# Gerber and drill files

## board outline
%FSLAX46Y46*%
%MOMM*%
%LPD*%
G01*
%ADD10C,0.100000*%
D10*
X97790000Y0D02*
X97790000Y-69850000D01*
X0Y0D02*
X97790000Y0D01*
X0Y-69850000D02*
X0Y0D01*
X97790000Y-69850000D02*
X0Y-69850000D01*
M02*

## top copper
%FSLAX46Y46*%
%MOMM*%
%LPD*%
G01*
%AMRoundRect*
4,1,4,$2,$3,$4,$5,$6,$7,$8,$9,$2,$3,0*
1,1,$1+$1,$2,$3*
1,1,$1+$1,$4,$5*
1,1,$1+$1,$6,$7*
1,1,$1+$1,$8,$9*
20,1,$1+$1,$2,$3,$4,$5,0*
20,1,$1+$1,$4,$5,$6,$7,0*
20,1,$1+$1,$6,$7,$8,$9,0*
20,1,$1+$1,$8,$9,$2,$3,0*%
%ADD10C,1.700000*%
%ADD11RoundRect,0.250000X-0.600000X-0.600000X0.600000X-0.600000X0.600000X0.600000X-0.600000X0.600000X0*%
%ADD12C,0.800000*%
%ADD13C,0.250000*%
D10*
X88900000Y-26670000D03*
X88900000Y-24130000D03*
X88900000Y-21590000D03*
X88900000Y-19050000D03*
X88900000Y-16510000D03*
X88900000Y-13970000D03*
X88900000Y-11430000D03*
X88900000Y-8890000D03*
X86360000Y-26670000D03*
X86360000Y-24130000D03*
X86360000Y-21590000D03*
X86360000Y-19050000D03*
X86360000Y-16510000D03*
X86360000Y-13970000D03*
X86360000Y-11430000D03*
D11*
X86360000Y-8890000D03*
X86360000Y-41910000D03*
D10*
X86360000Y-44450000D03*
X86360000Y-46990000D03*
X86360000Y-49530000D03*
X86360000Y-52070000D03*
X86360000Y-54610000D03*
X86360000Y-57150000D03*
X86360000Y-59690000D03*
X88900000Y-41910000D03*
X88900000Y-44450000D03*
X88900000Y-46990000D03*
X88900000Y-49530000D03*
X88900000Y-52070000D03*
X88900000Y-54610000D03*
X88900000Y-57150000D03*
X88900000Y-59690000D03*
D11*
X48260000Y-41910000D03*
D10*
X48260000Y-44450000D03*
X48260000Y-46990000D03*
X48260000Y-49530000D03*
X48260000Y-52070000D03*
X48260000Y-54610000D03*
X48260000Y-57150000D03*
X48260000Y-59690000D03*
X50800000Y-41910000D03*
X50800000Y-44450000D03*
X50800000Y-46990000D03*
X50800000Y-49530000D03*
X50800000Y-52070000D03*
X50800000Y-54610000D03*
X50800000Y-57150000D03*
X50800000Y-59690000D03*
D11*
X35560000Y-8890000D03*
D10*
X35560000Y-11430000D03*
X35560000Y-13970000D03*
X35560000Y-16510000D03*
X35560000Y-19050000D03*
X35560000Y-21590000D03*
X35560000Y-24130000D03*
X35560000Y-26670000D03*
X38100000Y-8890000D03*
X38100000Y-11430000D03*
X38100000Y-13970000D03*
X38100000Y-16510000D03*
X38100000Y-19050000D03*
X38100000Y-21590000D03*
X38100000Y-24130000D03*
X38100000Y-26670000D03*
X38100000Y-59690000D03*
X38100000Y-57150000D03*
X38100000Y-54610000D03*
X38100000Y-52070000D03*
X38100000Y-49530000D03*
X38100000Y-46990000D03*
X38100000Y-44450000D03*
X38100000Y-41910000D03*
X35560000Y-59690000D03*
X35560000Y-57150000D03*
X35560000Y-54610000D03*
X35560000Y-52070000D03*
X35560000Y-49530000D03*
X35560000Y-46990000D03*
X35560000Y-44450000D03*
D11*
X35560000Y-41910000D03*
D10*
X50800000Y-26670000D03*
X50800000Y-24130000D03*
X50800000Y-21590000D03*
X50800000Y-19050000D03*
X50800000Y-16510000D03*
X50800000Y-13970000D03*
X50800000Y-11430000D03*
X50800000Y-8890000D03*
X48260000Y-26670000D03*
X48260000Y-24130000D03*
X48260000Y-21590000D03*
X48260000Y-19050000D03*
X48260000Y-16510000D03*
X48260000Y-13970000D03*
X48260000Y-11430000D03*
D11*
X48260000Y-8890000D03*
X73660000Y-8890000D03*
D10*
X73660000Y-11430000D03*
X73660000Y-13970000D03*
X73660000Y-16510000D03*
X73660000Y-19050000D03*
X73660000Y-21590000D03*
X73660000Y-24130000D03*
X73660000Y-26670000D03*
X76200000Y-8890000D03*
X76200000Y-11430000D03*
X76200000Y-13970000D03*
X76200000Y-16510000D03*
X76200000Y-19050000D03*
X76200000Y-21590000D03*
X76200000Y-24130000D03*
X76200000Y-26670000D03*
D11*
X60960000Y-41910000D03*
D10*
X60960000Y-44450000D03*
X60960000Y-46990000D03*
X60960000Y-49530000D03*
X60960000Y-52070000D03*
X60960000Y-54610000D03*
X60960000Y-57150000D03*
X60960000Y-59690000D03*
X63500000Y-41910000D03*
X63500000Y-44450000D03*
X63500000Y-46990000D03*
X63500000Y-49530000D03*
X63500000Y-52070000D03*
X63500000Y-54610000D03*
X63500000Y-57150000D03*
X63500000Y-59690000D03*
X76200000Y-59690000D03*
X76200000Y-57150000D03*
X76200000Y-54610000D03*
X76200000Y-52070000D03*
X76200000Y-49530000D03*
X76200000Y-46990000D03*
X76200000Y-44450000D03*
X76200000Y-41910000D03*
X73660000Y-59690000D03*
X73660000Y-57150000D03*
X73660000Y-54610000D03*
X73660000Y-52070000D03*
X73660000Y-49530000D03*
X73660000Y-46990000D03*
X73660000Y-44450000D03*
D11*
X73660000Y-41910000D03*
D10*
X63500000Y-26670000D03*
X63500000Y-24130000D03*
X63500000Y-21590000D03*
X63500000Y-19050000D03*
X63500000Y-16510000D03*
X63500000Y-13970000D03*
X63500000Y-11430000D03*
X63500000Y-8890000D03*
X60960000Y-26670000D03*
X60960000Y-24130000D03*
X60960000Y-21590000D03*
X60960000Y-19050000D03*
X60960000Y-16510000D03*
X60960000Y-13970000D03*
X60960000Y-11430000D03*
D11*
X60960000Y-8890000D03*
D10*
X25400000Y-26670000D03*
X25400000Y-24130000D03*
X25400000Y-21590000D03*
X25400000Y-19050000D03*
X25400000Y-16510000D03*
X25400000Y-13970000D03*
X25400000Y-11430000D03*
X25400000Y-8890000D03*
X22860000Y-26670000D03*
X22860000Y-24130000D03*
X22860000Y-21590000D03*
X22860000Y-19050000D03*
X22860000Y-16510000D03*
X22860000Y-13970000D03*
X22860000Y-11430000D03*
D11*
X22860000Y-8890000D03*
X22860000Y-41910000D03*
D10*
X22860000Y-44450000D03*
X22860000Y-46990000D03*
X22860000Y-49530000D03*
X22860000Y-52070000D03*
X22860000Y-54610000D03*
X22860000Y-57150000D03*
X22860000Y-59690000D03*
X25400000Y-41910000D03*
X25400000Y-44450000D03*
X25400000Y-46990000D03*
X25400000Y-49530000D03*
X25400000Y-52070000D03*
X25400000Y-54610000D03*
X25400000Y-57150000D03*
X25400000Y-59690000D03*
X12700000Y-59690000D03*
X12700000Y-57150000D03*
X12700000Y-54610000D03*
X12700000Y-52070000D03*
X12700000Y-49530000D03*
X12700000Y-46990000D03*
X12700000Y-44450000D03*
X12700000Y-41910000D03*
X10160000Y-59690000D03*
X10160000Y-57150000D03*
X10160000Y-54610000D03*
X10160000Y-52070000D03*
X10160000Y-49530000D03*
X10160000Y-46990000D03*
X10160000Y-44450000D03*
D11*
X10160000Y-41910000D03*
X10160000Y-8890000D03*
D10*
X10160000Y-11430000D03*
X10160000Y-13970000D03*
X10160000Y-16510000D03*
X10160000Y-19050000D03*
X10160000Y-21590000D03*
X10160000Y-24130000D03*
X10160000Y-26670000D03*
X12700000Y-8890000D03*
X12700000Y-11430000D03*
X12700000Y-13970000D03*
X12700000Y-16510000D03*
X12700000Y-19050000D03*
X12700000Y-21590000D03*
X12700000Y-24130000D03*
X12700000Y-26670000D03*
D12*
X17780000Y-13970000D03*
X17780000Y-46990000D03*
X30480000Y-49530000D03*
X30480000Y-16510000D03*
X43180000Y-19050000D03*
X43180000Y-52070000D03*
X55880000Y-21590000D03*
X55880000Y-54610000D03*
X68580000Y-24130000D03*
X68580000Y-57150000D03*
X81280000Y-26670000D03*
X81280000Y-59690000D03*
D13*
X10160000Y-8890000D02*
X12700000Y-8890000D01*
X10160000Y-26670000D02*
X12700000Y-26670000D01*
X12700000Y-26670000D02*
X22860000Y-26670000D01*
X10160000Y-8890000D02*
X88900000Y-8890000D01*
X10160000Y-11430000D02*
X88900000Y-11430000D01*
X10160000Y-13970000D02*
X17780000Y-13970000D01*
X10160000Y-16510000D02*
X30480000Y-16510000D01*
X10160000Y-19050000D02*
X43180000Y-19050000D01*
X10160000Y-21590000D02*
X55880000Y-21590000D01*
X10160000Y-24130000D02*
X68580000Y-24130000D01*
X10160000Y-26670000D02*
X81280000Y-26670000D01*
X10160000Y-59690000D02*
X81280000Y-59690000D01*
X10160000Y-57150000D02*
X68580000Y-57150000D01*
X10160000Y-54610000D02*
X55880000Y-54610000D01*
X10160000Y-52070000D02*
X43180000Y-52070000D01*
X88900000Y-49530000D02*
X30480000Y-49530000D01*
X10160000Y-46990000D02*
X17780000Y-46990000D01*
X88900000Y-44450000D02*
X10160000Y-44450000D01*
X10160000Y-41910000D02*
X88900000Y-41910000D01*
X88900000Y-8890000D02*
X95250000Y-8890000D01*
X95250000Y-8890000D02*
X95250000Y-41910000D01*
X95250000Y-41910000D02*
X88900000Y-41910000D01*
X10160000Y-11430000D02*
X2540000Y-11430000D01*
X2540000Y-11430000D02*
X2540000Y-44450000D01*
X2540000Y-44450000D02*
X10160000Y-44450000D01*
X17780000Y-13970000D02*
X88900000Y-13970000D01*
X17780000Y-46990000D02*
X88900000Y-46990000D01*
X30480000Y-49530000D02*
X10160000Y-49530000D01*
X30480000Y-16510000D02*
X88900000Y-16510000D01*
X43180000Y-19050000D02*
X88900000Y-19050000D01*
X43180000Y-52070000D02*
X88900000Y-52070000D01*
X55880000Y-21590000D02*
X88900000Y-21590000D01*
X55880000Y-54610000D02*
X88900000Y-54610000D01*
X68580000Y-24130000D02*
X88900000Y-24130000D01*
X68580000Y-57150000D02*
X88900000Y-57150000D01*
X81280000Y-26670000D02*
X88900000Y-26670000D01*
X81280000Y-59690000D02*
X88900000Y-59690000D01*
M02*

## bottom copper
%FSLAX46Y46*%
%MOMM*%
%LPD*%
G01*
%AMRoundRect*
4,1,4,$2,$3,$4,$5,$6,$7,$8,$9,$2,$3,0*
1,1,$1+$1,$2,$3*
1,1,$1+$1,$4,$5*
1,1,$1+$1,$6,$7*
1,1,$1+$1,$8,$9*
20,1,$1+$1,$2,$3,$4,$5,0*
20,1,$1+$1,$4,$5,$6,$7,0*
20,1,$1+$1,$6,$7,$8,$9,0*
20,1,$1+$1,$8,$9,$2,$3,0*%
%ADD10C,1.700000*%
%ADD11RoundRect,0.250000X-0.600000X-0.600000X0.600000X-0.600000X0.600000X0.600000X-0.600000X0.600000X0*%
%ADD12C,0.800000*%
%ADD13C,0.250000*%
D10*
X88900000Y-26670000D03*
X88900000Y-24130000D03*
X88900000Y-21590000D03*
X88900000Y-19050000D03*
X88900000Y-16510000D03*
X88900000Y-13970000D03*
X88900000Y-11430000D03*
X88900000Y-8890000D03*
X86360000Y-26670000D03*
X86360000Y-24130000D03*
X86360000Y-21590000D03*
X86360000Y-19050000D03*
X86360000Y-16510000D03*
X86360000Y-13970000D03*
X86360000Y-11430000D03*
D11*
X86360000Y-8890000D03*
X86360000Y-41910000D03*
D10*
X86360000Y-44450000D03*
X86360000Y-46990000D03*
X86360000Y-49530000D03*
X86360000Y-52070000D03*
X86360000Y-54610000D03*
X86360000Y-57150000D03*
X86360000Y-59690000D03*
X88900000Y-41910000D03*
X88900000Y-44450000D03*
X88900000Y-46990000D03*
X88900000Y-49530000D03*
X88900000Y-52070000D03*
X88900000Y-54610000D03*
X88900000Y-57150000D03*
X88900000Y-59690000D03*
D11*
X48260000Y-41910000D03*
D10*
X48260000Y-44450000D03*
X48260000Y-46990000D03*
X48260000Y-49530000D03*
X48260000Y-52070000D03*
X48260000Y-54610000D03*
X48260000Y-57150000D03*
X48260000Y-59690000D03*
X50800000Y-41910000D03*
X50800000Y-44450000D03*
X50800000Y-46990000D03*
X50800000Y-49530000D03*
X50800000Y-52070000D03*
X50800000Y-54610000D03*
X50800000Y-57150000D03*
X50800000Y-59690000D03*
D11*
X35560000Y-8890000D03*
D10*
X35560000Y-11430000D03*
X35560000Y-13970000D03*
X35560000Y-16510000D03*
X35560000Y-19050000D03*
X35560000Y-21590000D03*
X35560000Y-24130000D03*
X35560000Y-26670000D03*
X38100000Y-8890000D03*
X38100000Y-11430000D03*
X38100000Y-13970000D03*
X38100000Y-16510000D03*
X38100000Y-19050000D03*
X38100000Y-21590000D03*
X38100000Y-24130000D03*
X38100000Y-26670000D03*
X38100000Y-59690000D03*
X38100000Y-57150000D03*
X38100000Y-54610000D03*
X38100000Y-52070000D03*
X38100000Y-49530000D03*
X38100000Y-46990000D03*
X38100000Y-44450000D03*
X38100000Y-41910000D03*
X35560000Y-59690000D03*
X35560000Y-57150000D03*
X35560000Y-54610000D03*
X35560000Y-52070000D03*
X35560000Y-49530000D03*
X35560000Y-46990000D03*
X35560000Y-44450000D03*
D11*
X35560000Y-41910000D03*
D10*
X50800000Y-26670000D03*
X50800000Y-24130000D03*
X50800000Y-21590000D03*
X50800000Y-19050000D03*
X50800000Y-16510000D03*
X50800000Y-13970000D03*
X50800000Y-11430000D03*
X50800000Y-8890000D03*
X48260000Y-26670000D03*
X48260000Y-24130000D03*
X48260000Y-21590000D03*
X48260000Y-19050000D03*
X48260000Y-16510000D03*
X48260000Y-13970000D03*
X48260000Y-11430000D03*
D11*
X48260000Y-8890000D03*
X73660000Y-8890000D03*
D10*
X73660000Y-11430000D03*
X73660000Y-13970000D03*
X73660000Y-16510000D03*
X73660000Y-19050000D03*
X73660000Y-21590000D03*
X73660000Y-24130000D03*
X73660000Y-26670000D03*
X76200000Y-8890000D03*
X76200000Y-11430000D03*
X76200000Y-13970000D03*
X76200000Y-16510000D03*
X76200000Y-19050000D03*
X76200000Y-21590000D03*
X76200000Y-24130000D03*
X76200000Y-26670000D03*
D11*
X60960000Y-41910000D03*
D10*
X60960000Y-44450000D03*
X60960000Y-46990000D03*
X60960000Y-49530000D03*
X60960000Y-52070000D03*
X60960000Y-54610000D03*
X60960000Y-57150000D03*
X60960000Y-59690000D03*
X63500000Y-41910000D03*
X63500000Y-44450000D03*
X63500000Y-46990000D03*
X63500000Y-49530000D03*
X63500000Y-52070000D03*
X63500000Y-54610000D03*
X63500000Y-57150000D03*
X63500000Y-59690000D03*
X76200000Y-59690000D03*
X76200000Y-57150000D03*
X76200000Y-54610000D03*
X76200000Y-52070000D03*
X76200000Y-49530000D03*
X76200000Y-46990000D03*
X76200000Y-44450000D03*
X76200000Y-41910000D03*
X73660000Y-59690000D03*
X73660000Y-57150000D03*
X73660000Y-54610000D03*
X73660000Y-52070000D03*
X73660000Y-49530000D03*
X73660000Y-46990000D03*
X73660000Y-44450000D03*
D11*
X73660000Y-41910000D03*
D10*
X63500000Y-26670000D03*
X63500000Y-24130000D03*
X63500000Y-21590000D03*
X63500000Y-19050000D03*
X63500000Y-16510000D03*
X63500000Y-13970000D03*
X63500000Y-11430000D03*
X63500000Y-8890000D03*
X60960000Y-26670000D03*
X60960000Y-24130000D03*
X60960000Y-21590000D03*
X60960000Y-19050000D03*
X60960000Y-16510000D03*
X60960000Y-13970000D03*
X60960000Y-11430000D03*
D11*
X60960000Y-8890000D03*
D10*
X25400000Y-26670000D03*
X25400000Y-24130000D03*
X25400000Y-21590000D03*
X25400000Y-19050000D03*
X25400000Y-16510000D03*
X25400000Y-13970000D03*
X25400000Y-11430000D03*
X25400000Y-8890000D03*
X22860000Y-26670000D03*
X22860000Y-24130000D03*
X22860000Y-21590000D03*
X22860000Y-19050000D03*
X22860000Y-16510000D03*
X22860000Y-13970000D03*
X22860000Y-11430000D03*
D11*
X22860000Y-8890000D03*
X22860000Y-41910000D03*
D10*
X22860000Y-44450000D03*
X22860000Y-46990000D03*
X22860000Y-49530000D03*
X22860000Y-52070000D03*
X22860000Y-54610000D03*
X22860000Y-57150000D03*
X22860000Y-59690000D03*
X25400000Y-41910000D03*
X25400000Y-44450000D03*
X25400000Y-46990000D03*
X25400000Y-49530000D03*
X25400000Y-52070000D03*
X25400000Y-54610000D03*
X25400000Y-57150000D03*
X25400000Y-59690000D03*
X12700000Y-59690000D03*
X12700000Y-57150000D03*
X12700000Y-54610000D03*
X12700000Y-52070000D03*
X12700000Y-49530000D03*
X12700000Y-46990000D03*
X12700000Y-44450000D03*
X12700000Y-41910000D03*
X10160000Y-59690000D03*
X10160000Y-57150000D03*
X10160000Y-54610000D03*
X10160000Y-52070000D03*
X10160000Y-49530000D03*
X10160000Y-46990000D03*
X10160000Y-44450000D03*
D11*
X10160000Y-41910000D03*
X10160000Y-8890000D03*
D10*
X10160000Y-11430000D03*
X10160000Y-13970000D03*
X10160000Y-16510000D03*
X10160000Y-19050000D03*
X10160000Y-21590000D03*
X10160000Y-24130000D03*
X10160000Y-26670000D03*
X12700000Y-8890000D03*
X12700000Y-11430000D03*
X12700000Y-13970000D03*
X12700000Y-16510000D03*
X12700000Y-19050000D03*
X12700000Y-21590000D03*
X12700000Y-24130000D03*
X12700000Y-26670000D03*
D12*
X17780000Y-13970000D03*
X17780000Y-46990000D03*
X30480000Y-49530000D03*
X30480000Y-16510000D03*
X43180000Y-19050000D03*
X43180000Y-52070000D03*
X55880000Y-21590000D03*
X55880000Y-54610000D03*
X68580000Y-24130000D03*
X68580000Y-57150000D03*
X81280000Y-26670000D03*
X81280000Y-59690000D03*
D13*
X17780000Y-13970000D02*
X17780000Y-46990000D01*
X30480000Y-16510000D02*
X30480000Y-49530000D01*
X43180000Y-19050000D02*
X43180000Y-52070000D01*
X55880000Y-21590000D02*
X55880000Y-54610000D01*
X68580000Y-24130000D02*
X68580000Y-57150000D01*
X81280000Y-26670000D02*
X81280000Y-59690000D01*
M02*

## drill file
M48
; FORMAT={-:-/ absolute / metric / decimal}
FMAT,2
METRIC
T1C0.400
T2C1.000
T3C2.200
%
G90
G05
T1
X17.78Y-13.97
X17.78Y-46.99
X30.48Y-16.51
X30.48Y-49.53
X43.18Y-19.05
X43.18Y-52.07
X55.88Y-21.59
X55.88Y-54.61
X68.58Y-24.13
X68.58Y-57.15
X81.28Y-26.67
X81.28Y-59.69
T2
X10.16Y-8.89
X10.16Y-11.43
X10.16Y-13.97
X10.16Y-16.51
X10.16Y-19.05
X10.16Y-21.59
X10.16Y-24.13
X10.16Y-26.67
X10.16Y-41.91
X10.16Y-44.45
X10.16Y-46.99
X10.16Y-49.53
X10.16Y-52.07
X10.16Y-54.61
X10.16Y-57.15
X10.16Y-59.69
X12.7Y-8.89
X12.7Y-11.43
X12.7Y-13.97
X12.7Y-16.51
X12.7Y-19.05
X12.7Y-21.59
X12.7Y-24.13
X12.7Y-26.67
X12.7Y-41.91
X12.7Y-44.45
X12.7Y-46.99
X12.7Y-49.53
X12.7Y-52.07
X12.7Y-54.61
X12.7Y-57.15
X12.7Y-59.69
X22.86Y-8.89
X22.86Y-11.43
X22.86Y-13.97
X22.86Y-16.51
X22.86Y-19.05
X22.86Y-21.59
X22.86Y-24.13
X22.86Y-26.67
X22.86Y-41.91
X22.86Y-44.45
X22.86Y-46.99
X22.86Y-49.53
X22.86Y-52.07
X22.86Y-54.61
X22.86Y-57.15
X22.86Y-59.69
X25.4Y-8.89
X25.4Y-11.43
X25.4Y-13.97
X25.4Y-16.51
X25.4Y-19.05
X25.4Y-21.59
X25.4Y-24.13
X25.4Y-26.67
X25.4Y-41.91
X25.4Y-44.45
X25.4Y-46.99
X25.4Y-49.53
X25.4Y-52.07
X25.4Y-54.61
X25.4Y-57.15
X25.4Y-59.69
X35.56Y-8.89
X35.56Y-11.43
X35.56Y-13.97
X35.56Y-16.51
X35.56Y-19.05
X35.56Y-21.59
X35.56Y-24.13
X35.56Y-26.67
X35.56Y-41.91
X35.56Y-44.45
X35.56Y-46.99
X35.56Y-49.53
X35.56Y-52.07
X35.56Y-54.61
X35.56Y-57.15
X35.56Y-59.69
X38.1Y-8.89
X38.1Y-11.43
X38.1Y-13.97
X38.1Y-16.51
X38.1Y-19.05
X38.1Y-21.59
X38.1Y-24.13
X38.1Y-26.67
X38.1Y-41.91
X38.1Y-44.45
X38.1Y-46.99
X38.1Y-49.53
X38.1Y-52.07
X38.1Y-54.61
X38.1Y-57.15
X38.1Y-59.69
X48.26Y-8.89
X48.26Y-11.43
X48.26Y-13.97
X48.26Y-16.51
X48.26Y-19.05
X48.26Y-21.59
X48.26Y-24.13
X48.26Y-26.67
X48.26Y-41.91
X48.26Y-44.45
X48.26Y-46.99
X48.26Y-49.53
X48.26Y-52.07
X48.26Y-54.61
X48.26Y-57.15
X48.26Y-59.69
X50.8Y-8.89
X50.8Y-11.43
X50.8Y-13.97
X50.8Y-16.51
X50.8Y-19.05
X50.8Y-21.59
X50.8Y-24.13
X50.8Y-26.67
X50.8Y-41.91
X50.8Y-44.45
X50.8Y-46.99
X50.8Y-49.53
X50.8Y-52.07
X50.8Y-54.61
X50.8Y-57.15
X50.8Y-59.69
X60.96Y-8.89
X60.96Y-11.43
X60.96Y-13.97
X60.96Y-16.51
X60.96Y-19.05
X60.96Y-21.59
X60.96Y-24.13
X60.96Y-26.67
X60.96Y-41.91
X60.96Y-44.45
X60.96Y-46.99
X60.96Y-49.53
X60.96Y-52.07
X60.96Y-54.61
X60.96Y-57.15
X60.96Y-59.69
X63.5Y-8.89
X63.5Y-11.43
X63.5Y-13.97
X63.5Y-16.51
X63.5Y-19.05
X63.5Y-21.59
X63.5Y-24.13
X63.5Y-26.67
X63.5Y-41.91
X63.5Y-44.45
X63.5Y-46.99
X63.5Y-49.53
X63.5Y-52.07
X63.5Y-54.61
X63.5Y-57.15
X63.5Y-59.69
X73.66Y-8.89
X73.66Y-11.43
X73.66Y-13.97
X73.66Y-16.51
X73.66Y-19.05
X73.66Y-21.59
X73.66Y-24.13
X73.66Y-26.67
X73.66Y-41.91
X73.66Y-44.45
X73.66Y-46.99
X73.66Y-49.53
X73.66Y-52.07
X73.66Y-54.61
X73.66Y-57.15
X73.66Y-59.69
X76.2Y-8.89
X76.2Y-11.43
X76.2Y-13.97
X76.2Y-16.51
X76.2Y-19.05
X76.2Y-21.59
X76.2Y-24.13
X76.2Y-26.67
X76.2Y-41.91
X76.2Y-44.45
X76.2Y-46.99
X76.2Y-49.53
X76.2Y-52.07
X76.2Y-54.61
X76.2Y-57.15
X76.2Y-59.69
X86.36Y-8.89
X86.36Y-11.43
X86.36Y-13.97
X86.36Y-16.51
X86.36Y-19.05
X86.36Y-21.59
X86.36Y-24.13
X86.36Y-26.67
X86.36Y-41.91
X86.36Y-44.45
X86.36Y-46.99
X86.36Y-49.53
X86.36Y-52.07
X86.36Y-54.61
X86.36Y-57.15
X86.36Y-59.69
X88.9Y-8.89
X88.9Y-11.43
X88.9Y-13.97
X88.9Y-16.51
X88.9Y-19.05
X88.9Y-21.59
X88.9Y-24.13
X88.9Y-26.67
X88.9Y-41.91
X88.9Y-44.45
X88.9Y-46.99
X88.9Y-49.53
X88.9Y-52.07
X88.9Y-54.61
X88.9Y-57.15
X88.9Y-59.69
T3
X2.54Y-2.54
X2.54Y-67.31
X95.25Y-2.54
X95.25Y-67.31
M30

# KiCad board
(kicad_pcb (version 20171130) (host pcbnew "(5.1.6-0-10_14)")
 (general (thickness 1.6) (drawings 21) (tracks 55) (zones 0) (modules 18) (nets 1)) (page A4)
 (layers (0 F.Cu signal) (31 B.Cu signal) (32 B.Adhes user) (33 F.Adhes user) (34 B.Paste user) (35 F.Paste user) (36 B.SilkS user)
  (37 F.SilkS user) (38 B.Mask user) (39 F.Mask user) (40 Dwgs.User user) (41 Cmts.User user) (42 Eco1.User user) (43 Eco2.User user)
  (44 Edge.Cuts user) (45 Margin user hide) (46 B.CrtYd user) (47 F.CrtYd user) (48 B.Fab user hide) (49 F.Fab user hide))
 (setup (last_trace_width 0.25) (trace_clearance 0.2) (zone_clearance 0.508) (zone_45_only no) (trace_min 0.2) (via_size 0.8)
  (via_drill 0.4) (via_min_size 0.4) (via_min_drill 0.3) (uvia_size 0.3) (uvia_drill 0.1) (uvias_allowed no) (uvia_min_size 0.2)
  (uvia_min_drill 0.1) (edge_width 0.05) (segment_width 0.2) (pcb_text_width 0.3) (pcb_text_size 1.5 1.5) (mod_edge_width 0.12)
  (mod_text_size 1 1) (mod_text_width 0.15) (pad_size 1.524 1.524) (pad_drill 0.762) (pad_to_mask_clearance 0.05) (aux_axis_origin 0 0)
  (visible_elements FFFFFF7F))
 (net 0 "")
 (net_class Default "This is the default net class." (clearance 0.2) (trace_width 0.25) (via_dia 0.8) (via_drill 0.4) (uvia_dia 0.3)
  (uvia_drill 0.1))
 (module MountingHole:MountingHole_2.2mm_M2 (layer F.Cu) (at 95.25 2.54)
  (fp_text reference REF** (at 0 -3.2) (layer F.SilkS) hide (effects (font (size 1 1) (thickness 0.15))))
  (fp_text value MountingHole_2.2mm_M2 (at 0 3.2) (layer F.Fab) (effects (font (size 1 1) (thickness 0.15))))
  (pad 1 np_thru_hole circle (at 0 0) (size 2.2 2.2) (drill 2.2) (layers *.Cu *.Mask)))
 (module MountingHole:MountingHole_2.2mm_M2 (layer F.Cu) (at 2.54 2.54)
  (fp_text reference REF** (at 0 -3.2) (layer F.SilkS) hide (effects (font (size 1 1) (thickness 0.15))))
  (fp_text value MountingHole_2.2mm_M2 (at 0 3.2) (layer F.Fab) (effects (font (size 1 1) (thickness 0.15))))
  (pad 1 np_thru_hole circle (at 0 0) (size 2.2 2.2) (drill 2.2) (layers *.Cu *.Mask)))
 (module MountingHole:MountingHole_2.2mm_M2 (layer F.Cu) (at 2.54 67.31)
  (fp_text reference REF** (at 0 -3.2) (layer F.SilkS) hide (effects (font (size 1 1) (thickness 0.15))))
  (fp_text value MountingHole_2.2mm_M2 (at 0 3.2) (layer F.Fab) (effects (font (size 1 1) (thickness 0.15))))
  (pad 1 np_thru_hole circle (at 0 0) (size 2.2 2.2) (drill 2.2) (layers *.Cu *.Mask)))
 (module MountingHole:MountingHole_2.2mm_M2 (layer F.Cu) (at 95.25 67.31)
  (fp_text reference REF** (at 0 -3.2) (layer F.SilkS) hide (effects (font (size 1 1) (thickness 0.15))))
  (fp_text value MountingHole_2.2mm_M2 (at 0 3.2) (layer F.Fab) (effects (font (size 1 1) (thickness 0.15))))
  (pad 1 np_thru_hole circle (at 0 0) (size 2.2 2.2) (drill 2.2) (layers *.Cu *.Mask)))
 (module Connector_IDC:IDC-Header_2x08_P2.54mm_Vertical (layer F.Cu) (at 86.36 8.89)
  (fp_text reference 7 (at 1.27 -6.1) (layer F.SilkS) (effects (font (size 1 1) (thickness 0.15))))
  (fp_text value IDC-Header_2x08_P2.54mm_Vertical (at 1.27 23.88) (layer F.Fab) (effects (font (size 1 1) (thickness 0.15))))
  (pad 16 thru_hole circle (at 2.54 17.78) (size 1.7 1.7) (drill 1) (layers *.Cu *.Mask))
  (pad 14 thru_hole circle (at 2.54 15.24) (size 1.7 1.7) (drill 1) (layers *.Cu *.Mask))
  (pad 12 thru_hole circle (at 2.54 12.7) (size 1.7 1.7) (drill 1) (layers *.Cu *.Mask))
  (pad 10 thru_hole circle (at 2.54 10.16) (size 1.7 1.7) (drill 1) (layers *.Cu *.Mask))
  (pad 8 thru_hole circle (at 2.54 7.62) (size 1.7 1.7) (drill 1) (layers *.Cu *.Mask))
  (pad 6 thru_hole circle (at 2.54 5.08) (size 1.7 1.7) (drill 1) (layers *.Cu *.Mask))
  (pad 4 thru_hole circle (at 2.54 2.54) (size 1.7 1.7) (drill 1) (layers *.Cu *.Mask))
  (pad 2 thru_hole circle (at 2.54 0) (size 1.7 1.7) (drill 1) (layers *.Cu *.Mask))
  (pad 15 thru_hole circle (at 0 17.78) (size 1.7 1.7) (drill 1) (layers *.Cu *.Mask))
  (pad 13 thru_hole circle (at 0 15.24) (size 1.7 1.7) (drill 1) (layers *.Cu *.Mask))
  (pad 11 thru_hole circle (at 0 12.7) (size 1.7 1.7) (drill 1) (layers *.Cu *.Mask))
  (pad 9 thru_hole circle (at 0 10.16) (size 1.7 1.7) (drill 1) (layers *.Cu *.Mask))
  (pad 7 thru_hole circle (at 0 7.62) (size 1.7 1.7) (drill 1) (layers *.Cu *.Mask))
  (pad 5 thru_hole circle (at 0 5.08) (size 1.7 1.7) (drill 1) (layers *.Cu *.Mask))
  (pad 3 thru_hole circle (at 0 2.54) (size 1.7 1.7) (drill 1) (layers *.Cu *.Mask))
  (pad 1 thru_hole roundrect (at 0 0) (size 1.7 1.7) (drill 1) (layers *.Cu *.Mask) (roundrect_rratio 0.147059)))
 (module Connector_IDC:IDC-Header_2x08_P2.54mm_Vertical (layer F.Cu) (at 86.36 41.91)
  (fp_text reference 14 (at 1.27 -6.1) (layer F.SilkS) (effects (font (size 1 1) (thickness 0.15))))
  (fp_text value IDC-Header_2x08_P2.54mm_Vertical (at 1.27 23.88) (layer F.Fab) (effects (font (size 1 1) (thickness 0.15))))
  (pad 1 thru_hole roundrect (at 0 0) (size 1.7 1.7) (drill 1) (layers *.Cu *.Mask) (roundrect_rratio 0.147059))
  (pad 3 thru_hole circle (at 0 2.54) (size 1.7 1.7) (drill 1) (layers *.Cu *.Mask))
  (pad 5 thru_hole circle (at 0 5.08) (size 1.7 1.7) (drill 1) (layers *.Cu *.Mask))
  (pad 7 thru_hole circle (at 0 7.62) (size 1.7 1.7) (drill 1) (layers *.Cu *.Mask))
  (pad 9 thru_hole circle (at 0 10.16) (size 1.7 1.7) (drill 1) (layers *.Cu *.Mask))
  (pad 11 thru_hole circle (at 0 12.7) (size 1.7 1.7) (drill 1) (layers *.Cu *.Mask))
  (pad 13 thru_hole circle (at 0 15.24) (size 1.7 1.7) (drill 1) (layers *.Cu *.Mask))
  (pad 15 thru_hole circle (at 0 17.78) (size 1.7 1.7) (drill 1) (layers *.Cu *.Mask))
  (pad 2 thru_hole circle (at 2.54 0) (size 1.7 1.7) (drill 1) (layers *.Cu *.Mask))
  (pad 4 thru_hole circle (at 2.54 2.54) (size 1.7 1.7) (drill 1) (layers *.Cu *.Mask))
  (pad 6 thru_hole circle (at 2.54 5.08) (size 1.7 1.7) (drill 1) (layers *.Cu *.Mask))
  (pad 8 thru_hole circle (at 2.54 7.62) (size 1.7 1.7) (drill 1) (layers *.Cu *.Mask))
  (pad 10 thru_hole circle (at 2.54 10.16) (size 1.7 1.7) (drill 1) (layers *.Cu *.Mask))
  (pad 12 thru_hole circle (at 2.54 12.7) (size 1.7 1.7) (drill 1) (layers *.Cu *.Mask))
  (pad 14 thru_hole circle (at 2.54 15.24) (size 1.7 1.7) (drill 1) (layers *.Cu *.Mask))
  (pad 16 thru_hole circle (at 2.54 17.78) (size 1.7 1.7) (drill 1) (layers *.Cu *.Mask)))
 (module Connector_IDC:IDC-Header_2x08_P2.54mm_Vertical (layer F.Cu) (at 48.26 41.91)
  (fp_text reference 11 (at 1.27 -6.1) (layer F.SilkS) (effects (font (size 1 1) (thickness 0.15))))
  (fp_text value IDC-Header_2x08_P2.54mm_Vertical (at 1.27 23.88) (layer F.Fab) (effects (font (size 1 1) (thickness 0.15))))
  (pad 1 thru_hole roundrect (at 0 0) (size 1.7 1.7) (drill 1) (layers *.Cu *.Mask) (roundrect_rratio 0.147059))
  (pad 3 thru_hole circle (at 0 2.54) (size 1.7 1.7) (drill 1) (layers *.Cu *.Mask))
  (pad 5 thru_hole circle (at 0 5.08) (size 1.7 1.7) (drill 1) (layers *.Cu *.Mask))
  (pad 7 thru_hole circle (at 0 7.62) (size 1.7 1.7) (drill 1) (layers *.Cu *.Mask))
  (pad 9 thru_hole circle (at 0 10.16) (size 1.7 1.7) (drill 1) (layers *.Cu *.Mask))
  (pad 11 thru_hole circle (at 0 12.7) (size 1.7 1.7) (drill 1) (layers *.Cu *.Mask))
  (pad 13 thru_hole circle (at 0 15.24) (size 1.7 1.7) (drill 1) (layers *.Cu *.Mask))
  (pad 15 thru_hole circle (at 0 17.78) (size 1.7 1.7) (drill 1) (layers *.Cu *.Mask))
  (pad 2 thru_hole circle (at 2.54 0) (size 1.7 1.7) (drill 1) (layers *.Cu *.Mask))
  (pad 4 thru_hole circle (at 2.54 2.54) (size 1.7 1.7) (drill 1) (layers *.Cu *.Mask))
  (pad 6 thru_hole circle (at 2.54 5.08) (size 1.7 1.7) (drill 1) (layers *.Cu *.Mask))
  (pad 8 thru_hole circle (at 2.54 7.62) (size 1.7 1.7) (drill 1) (layers *.Cu *.Mask))
  (pad 10 thru_hole circle (at 2.54 10.16) (size 1.7 1.7) (drill 1) (layers *.Cu *.Mask))
  (pad 12 thru_hole circle (at 2.54 12.7) (size 1.7 1.7) (drill 1) (layers *.Cu *.Mask))
  (pad 14 thru_hole circle (at 2.54 15.24) (size 1.7 1.7) (drill 1) (layers *.Cu *.Mask))
  (pad 16 thru_hole circle (at 2.54 17.78) (size 1.7 1.7) (drill 1) (layers *.Cu *.Mask)))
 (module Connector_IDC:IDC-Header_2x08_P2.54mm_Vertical (layer F.Cu) (at 35.56 8.89)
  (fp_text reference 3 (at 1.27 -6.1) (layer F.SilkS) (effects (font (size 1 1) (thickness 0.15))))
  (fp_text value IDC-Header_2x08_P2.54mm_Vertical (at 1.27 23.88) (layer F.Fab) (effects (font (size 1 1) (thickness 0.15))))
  (pad 1 thru_hole roundrect (at 0 0) (size 1.7 1.7) (drill 1) (layers *.Cu *.Mask) (roundrect_rratio 0.147059))
  (pad 3 thru_hole circle (at 0 2.54) (size 1.7 1.7) (drill 1) (layers *.Cu *.Mask))
  (pad 5 thru_hole circle (at 0 5.08) (size 1.7 1.7) (drill 1) (layers *.Cu *.Mask))
  (pad 7 thru_hole circle (at 0 7.62) (size 1.7 1.7) (drill 1) (layers *.Cu *.Mask))
  (pad 9 thru_hole circle (at 0 10.16) (size 1.7 1.7) (drill 1) (layers *.Cu *.Mask))
  (pad 11 thru_hole circle (at 0 12.7) (size 1.7 1.7) (drill 1) (layers *.Cu *.Mask))
  (pad 13 thru_hole circle (at 0 15.24) (size 1.7 1.7) (drill 1) (layers *.Cu *.Mask))
  (pad 15 thru_hole circle (at 0 17.78) (size 1.7 1.7) (drill 1) (layers *.Cu *.Mask))
  (pad 2 thru_hole circle (at 2.54 0) (size 1.7 1.7) (drill 1) (layers *.Cu *.Mask))
  (pad 4 thru_hole circle (at 2.54 2.54) (size 1.7 1.7) (drill 1) (layers *.Cu *.Mask))
  (pad 6 thru_hole circle (at 2.54 5.08) (size 1.7 1.7) (drill 1) (layers *.Cu *.Mask))
  (pad 8 thru_hole circle (at 2.54 7.62) (size 1.7 1.7) (drill 1) (layers *.Cu *.Mask))
  (pad 10 thru_hole circle (at 2.54 10.16) (size 1.7 1.7) (drill 1) (layers *.Cu *.Mask))
  (pad 12 thru_hole circle (at 2.54 12.7) (size 1.7 1.7) (drill 1) (layers *.Cu *.Mask))
  (pad 14 thru_hole circle (at 2.54 15.24) (size 1.7 1.7) (drill 1) (layers *.Cu *.Mask))
  (pad 16 thru_hole circle (at 2.54 17.78) (size 1.7 1.7) (drill 1) (layers *.Cu *.Mask)))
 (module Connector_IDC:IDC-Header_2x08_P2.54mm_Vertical (layer F.Cu) (at 35.56 41.91)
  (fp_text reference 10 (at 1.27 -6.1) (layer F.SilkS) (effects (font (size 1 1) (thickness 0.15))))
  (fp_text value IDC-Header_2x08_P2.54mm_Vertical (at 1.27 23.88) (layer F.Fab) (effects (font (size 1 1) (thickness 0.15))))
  (pad 16 thru_hole circle (at 2.54 17.78) (size 1.7 1.7) (drill 1) (layers *.Cu *.Mask))
  (pad 14 thru_hole circle (at 2.54 15.24) (size 1.7 1.7) (drill 1) (layers *.Cu *.Mask))
  (pad 12 thru_hole circle (at 2.54 12.7) (size 1.7 1.7) (drill 1) (layers *.Cu *.Mask))
  (pad 10 thru_hole circle (at 2.54 10.16) (size 1.7 1.7) (drill 1) (layers *.Cu *.Mask))
  (pad 8 thru_hole circle (at 2.54 7.62) (size 1.7 1.7) (drill 1) (layers *.Cu *.Mask))
  (pad 6 thru_hole circle (at 2.54 5.08) (size 1.7 1.7) (drill 1) (layers *.Cu *.Mask))
  (pad 4 thru_hole circle (at 2.54 2.54) (size 1.7 1.7) (drill 1) (layers *.Cu *.Mask))
  (pad 2 thru_hole circle (at 2.54 0) (size 1.7 1.7) (drill 1) (layers *.Cu *.Mask))
  (pad 15 thru_hole circle (at 0 17.78) (size 1.7 1.7) (drill 1) (layers *.Cu *.Mask))
  (pad 13 thru_hole circle (at 0 15.24) (size 1.7 1.7) (drill 1) (layers *.Cu *.Mask))
  (pad 11 thru_hole circle (at 0 12.7) (size 1.7 1.7) (drill 1) (layers *.Cu *.Mask))
  (pad 9 thru_hole circle (at 0 10.16) (size 1.7 1.7) (drill 1) (layers *.Cu *.Mask))
  (pad 7 thru_hole circle (at 0 7.62) (size 1.7 1.7) (drill 1) (layers *.Cu *.Mask))
  (pad 5 thru_hole circle (at 0 5.08) (size 1.7 1.7) (drill 1) (layers *.Cu *.Mask))
  (pad 3 thru_hole circle (at 0 2.54) (size 1.7 1.7) (drill 1) (layers *.Cu *.Mask))
  (pad 1 thru_hole roundrect (at 0 0) (size 1.7 1.7) (drill 1) (layers *.Cu *.Mask) (roundrect_rratio 0.147059)))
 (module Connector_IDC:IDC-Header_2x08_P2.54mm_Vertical (layer F.Cu) (at 48.26 8.89)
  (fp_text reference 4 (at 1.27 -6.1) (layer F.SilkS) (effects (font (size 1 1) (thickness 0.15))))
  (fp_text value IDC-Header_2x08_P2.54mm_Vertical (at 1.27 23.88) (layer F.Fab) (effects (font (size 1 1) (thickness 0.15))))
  (pad 16 thru_hole circle (at 2.54 17.78) (size 1.7 1.7) (drill 1) (layers *.Cu *.Mask))
  (pad 14 thru_hole circle (at 2.54 15.24) (size 1.7 1.7) (drill 1) (layers *.Cu *.Mask))
  (pad 12 thru_hole circle (at 2.54 12.7) (size 1.7 1.7) (drill 1) (layers *.Cu *.Mask))
  (pad 10 thru_hole circle (at 2.54 10.16) (size 1.7 1.7) (drill 1) (layers *.Cu *.Mask))
  (pad 8 thru_hole circle (at 2.54 7.62) (size 1.7 1.7) (drill 1) (layers *.Cu *.Mask))
  (pad 6 thru_hole circle (at 2.54 5.08) (size 1.7 1.7) (drill 1) (layers *.Cu *.Mask))
  (pad 4 thru_hole circle (at 2.54 2.54) (size 1.7 1.7) (drill 1) (layers *.Cu *.Mask))
  (pad 2 thru_hole circle (at 2.54 0) (size 1.7 1.7) (drill 1) (layers *.Cu *.Mask))
  (pad 15 thru_hole circle (at 0 17.78) (size 1.7 1.7) (drill 1) (layers *.Cu *.Mask))
  (pad 13 thru_hole circle (at 0 15.24) (size 1.7 1.7) (drill 1) (layers *.Cu *.Mask))
  (pad 11 thru_hole circle (at 0 12.7) (size 1.7 1.7) (drill 1) (layers *.Cu *.Mask))
  (pad 9 thru_hole circle (at 0 10.16) (size 1.7 1.7) (drill 1) (layers *.Cu *.Mask))
  (pad 7 thru_hole circle (at 0 7.62) (size 1.7 1.7) (drill 1) (layers *.Cu *.Mask))
  (pad 5 thru_hole circle (at 0 5.08) (size 1.7 1.7) (drill 1) (layers *.Cu *.Mask))
  (pad 3 thru_hole circle (at 0 2.54) (size 1.7 1.7) (drill 1) (layers *.Cu *.Mask))
  (pad 1 thru_hole roundrect (at 0 0) (size 1.7 1.7) (drill 1) (layers *.Cu *.Mask) (roundrect_rratio 0.147059)))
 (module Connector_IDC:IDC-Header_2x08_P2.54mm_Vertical (layer F.Cu) (at 73.66 8.89)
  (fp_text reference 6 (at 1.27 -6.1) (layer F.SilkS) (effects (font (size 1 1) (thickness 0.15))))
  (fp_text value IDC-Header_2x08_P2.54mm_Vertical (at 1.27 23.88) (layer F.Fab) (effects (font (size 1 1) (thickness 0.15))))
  (pad 1 thru_hole roundrect (at 0 0) (size 1.7 1.7) (drill 1) (layers *.Cu *.Mask) (roundrect_rratio 0.147059))
  (pad 3 thru_hole circle (at 0 2.54) (size 1.7 1.7) (drill 1) (layers *.Cu *.Mask))
  (pad 5 thru_hole circle (at 0 5.08) (size 1.7 1.7) (drill 1) (layers *.Cu *.Mask))
  (pad 7 thru_hole circle (at 0 7.62) (size 1.7 1.7) (drill 1) (layers *.Cu *.Mask))
  (pad 9 thru_hole circle (at 0 10.16) (size 1.7 1.7) (drill 1) (layers *.Cu *.Mask))
  (pad 11 thru_hole circle (at 0 12.7) (size 1.7 1.7) (drill 1) (layers *.Cu *.Mask))
  (pad 13 thru_hole circle (at 0 15.24) (size 1.7 1.7) (drill 1) (layers *.Cu *.Mask))
  (pad 15 thru_hole circle (at 0 17.78) (size 1.7 1.7) (drill 1) (layers *.Cu *.Mask))
  (pad 2 thru_hole circle (at 2.54 0) (size 1.7 1.7) (drill 1) (layers *.Cu *.Mask))
  (pad 4 thru_hole circle (at 2.54 2.54) (size 1.7 1.7) (drill 1) (layers *.Cu *.Mask))
  (pad 6 thru_hole circle (at 2.54 5.08) (size 1.7 1.7) (drill 1) (layers *.Cu *.Mask))
  (pad 8 thru_hole circle (at 2.54 7.62) (size 1.7 1.7) (drill 1) (layers *.Cu *.Mask))
  (pad 10 thru_hole circle (at 2.54 10.16) (size 1.7 1.7) (drill 1) (layers *.Cu *.Mask))
  (pad 12 thru_hole circle (at 2.54 12.7) (size 1.7 1.7) (drill 1) (layers *.Cu *.Mask))
  (pad 14 thru_hole circle (at 2.54 15.24) (size 1.7 1.7) (drill 1) (layers *.Cu *.Mask))
  (pad 16 thru_hole circle (at 2.54 17.78) (size 1.7 1.7) (drill 1) (layers *.Cu *.Mask)))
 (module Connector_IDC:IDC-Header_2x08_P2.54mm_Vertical (layer F.Cu) (at 60.96 41.91)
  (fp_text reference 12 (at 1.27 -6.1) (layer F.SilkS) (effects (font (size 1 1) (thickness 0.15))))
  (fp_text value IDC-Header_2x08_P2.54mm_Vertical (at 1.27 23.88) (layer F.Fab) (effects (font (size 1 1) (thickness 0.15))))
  (pad 1 thru_hole roundrect (at 0 0) (size 1.7 1.7) (drill 1) (layers *.Cu *.Mask) (roundrect_rratio 0.147059))
  (pad 3 thru_hole circle (at 0 2.54) (size 1.7 1.7) (drill 1) (layers *.Cu *.Mask))
  (pad 5 thru_hole circle (at 0 5.08) (size 1.7 1.7) (drill 1) (layers *.Cu *.Mask))
  (pad 7 thru_hole circle (at 0 7.62) (size 1.7 1.7) (drill 1) (layers *.Cu *.Mask))
  (pad 9 thru_hole circle (at 0 10.16) (size 1.7 1.7) (drill 1) (layers *.Cu *.Mask))
  (pad 11 thru_hole circle (at 0 12.7) (size 1.7 1.7) (drill 1) (layers *.Cu *.Mask))
  (pad 13 thru_hole circle (at 0 15.24) (size 1.7 1.7) (drill 1) (layers *.Cu *.Mask))
  (pad 15 thru_hole circle (at 0 17.78) (size 1.7 1.7) (drill 1) (layers *.Cu *.Mask))
  (pad 2 thru_hole circle (at 2.54 0) (size 1.7 1.7) (drill 1) (layers *.Cu *.Mask))
  (pad 4 thru_hole circle (at 2.54 2.54) (size 1.7 1.7) (drill 1) (layers *.Cu *.Mask))
  (pad 6 thru_hole circle (at 2.54 5.08) (size 1.7 1.7) (drill 1) (layers *.Cu *.Mask))
  (pad 8 thru_hole circle (at 2.54 7.62) (size 1.7 1.7) (drill 1) (layers *.Cu *.Mask))
  (pad 10 thru_hole circle (at 2.54 10.16) (size 1.7 1.7) (drill 1) (layers *.Cu *.Mask))
  (pad 12 thru_hole circle (at 2.54 12.7) (size 1.7 1.7) (drill 1) (layers *.Cu *.Mask))
  (pad 14 thru_hole circle (at 2.54 15.24) (size 1.7 1.7) (drill 1) (layers *.Cu *.Mask))
  (pad 16 thru_hole circle (at 2.54 17.78) (size 1.7 1.7) (drill 1) (layers *.Cu *.Mask)))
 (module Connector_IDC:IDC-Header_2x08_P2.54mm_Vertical (layer F.Cu) (at 73.66 41.91)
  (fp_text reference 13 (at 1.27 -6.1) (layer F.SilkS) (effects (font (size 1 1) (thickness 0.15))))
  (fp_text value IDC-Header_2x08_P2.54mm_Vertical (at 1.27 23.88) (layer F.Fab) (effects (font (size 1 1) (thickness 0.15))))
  (pad 16 thru_hole circle (at 2.54 17.78) (size 1.7 1.7) (drill 1) (layers *.Cu *.Mask))
  (pad 14 thru_hole circle (at 2.54 15.24) (size 1.7 1.7) (drill 1) (layers *.Cu *.Mask))
  (pad 12 thru_hole circle (at 2.54 12.7) (size 1.7 1.7) (drill 1) (layers *.Cu *.Mask))
  (pad 10 thru_hole circle (at 2.54 10.16) (size 1.7 1.7) (drill 1) (layers *.Cu *.Mask))
  (pad 8 thru_hole circle (at 2.54 7.62) (size 1.7 1.7) (drill 1) (layers *.Cu *.Mask))
  (pad 6 thru_hole circle (at 2.54 5.08) (size 1.7 1.7) (drill 1) (layers *.Cu *.Mask))
  (pad 4 thru_hole circle (at 2.54 2.54) (size 1.7 1.7) (drill 1) (layers *.Cu *.Mask))
  (pad 2 thru_hole circle (at 2.54 0) (size 1.7 1.7) (drill 1) (layers *.Cu *.Mask))
  (pad 15 thru_hole circle (at 0 17.78) (size 1.7 1.7) (drill 1) (layers *.Cu *.Mask))
  (pad 13 thru_hole circle (at 0 15.24) (size 1.7 1.7) (drill 1) (layers *.Cu *.Mask))
  (pad 11 thru_hole circle (at 0 12.7) (size 1.7 1.7) (drill 1) (layers *.Cu *.Mask))
  (pad 9 thru_hole circle (at 0 10.16) (size 1.7 1.7) (drill 1) (layers *.Cu *.Mask))
  (pad 7 thru_hole circle (at 0 7.62) (size 1.7 1.7) (drill 1) (layers *.Cu *.Mask))
  (pad 5 thru_hole circle (at 0 5.08) (size 1.7 1.7) (drill 1) (layers *.Cu *.Mask))
  (pad 3 thru_hole circle (at 0 2.54) (size 1.7 1.7) (drill 1) (layers *.Cu *.Mask))
  (pad 1 thru_hole roundrect (at 0 0) (size 1.7 1.7) (drill 1) (layers *.Cu *.Mask) (roundrect_rratio 0.147059)))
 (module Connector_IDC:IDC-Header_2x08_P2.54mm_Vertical (layer F.Cu) (at 60.96 8.89)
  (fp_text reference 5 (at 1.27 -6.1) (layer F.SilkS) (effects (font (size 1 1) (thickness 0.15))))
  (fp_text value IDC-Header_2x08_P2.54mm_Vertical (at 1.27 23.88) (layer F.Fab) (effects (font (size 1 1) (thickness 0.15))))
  (pad 16 thru_hole circle (at 2.54 17.78) (size 1.7 1.7) (drill 1) (layers *.Cu *.Mask))
  (pad 14 thru_hole circle (at 2.54 15.24) (size 1.7 1.7) (drill 1) (layers *.Cu *.Mask))
  (pad 12 thru_hole circle (at 2.54 12.7) (size 1.7 1.7) (drill 1) (layers *.Cu *.Mask))
  (pad 10 thru_hole circle (at 2.54 10.16) (size 1.7 1.7) (drill 1) (layers *.Cu *.Mask))
  (pad 8 thru_hole circle (at 2.54 7.62) (size 1.7 1.7) (drill 1) (layers *.Cu *.Mask))
  (pad 6 thru_hole circle (at 2.54 5.08) (size 1.7 1.7) (drill 1) (layers *.Cu *.Mask))
  (pad 4 thru_hole circle (at 2.54 2.54) (size 1.7 1.7) (drill 1) (layers *.Cu *.Mask))
  (pad 2 thru_hole circle (at 2.54 0) (size 1.7 1.7) (drill 1) (layers *.Cu *.Mask))
  (pad 15 thru_hole circle (at 0 17.78) (size 1.7 1.7) (drill 1) (layers *.Cu *.Mask))
  (pad 13 thru_hole circle (at 0 15.24) (size 1.7 1.7) (drill 1) (layers *.Cu *.Mask))
  (pad 11 thru_hole circle (at 0 12.7) (size 1.7 1.7) (drill 1) (layers *.Cu *.Mask))
  (pad 9 thru_hole circle (at 0 10.16) (size 1.7 1.7) (drill 1) (layers *.Cu *.Mask))
  (pad 7 thru_hole circle (at 0 7.62) (size 1.7 1.7) (drill 1) (layers *.Cu *.Mask))
  (pad 5 thru_hole circle (at 0 5.08) (size 1.7 1.7) (drill 1) (layers *.Cu *.Mask))
  (pad 3 thru_hole circle (at 0 2.54) (size 1.7 1.7) (drill 1) (layers *.Cu *.Mask))
  (pad 1 thru_hole roundrect (at 0 0) (size 1.7 1.7) (drill 1) (layers *.Cu *.Mask) (roundrect_rratio 0.147059)))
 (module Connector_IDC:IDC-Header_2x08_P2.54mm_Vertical (layer F.Cu) (at 22.86 8.89)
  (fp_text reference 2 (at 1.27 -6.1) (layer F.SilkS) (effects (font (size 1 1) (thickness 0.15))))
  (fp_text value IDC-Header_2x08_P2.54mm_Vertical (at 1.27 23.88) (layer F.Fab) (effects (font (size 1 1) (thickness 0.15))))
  (pad 16 thru_hole circle (at 2.54 17.78) (size 1.7 1.7) (drill 1) (layers *.Cu *.Mask))
  (pad 14 thru_hole circle (at 2.54 15.24) (size 1.7 1.7) (drill 1) (layers *.Cu *.Mask))
  (pad 12 thru_hole circle (at 2.54 12.7) (size 1.7 1.7) (drill 1) (layers *.Cu *.Mask))
  (pad 10 thru_hole circle (at 2.54 10.16) (size 1.7 1.7) (drill 1) (layers *.Cu *.Mask))
  (pad 8 thru_hole circle (at 2.54 7.62) (size 1.7 1.7) (drill 1) (layers *.Cu *.Mask))
  (pad 6 thru_hole circle (at 2.54 5.08) (size 1.7 1.7) (drill 1) (layers *.Cu *.Mask))
  (pad 4 thru_hole circle (at 2.54 2.54) (size 1.7 1.7) (drill 1) (layers *.Cu *.Mask))
  (pad 2 thru_hole circle (at 2.54 0) (size 1.7 1.7) (drill 1) (layers *.Cu *.Mask))
  (pad 15 thru_hole circle (at 0 17.78) (size 1.7 1.7) (drill 1) (layers *.Cu *.Mask))
  (pad 13 thru_hole circle (at 0 15.24) (size 1.7 1.7) (drill 1) (layers *.Cu *.Mask))
  (pad 11 thru_hole circle (at 0 12.7) (size 1.7 1.7) (drill 1) (layers *.Cu *.Mask))
  (pad 9 thru_hole circle (at 0 10.16) (size 1.7 1.7) (drill 1) (layers *.Cu *.Mask))
  (pad 7 thru_hole circle (at 0 7.62) (size 1.7 1.7) (drill 1) (layers *.Cu *.Mask))
  (pad 5 thru_hole circle (at 0 5.08) (size 1.7 1.7) (drill 1) (layers *.Cu *.Mask))
  (pad 3 thru_hole circle (at 0 2.54) (size 1.7 1.7) (drill 1) (layers *.Cu *.Mask))
  (pad 1 thru_hole roundrect (at 0 0) (size 1.7 1.7) (drill 1) (layers *.Cu *.Mask) (roundrect_rratio 0.147059)))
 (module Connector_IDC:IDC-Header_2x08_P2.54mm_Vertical (layer F.Cu) (at 22.86 41.91)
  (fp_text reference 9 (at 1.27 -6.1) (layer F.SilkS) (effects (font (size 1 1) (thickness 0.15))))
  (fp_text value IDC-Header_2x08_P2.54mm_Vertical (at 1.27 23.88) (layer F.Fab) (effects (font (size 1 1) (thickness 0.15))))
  (pad 1 thru_hole roundrect (at 0 0) (size 1.7 1.7) (drill 1) (layers *.Cu *.Mask) (roundrect_rratio 0.147059))
  (pad 3 thru_hole circle (at 0 2.54) (size 1.7 1.7) (drill 1) (layers *.Cu *.Mask))
  (pad 5 thru_hole circle (at 0 5.08) (size 1.7 1.7) (drill 1) (layers *.Cu *.Mask))
  (pad 7 thru_hole circle (at 0 7.62) (size 1.7 1.7) (drill 1) (layers *.Cu *.Mask))
  (pad 9 thru_hole circle (at 0 10.16) (size 1.7 1.7) (drill 1) (layers *.Cu *.Mask))
  (pad 11 thru_hole circle (at 0 12.7) (size 1.7 1.7) (drill 1) (layers *.Cu *.Mask))
  (pad 13 thru_hole circle (at 0 15.24) (size 1.7 1.7) (drill 1) (layers *.Cu *.Mask))
  (pad 15 thru_hole circle (at 0 17.78) (size 1.7 1.7) (drill 1) (layers *.Cu *.Mask))
  (pad 2 thru_hole circle (at 2.54 0) (size 1.7 1.7) (drill 1) (layers *.Cu *.Mask))
  (pad 4 thru_hole circle (at 2.54 2.54) (size 1.7 1.7) (drill 1) (layers *.Cu *.Mask))
  (pad 6 thru_hole circle (at 2.54 5.08) (size 1.7 1.7) (drill 1) (layers *.Cu *.Mask))
  (pad 8 thru_hole circle (at 2.54 7.62) (size 1.7 1.7) (drill 1) (layers *.Cu *.Mask))
  (pad 10 thru_hole circle (at 2.54 10.16) (size 1.7 1.7) (drill 1) (layers *.Cu *.Mask))
  (pad 12 thru_hole circle (at 2.54 12.7) (size 1.7 1.7) (drill 1) (layers *.Cu *.Mask))
  (pad 14 thru_hole circle (at 2.54 15.24) (size 1.7 1.7) (drill 1) (layers *.Cu *.Mask))
  (pad 16 thru_hole circle (at 2.54 17.78) (size 1.7 1.7) (drill 1) (layers *.Cu *.Mask)))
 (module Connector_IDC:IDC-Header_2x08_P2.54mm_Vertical (layer F.Cu) (at 10.16 41.91)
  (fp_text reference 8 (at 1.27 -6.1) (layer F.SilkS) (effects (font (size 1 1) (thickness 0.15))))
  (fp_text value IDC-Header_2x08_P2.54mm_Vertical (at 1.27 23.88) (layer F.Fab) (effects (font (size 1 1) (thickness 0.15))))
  (pad 16 thru_hole circle (at 2.54 17.78) (size 1.7 1.7) (drill 1) (layers *.Cu *.Mask))
  (pad 14 thru_hole circle (at 2.54 15.24) (size 1.7 1.7) (drill 1) (layers *.Cu *.Mask))
  (pad 12 thru_hole circle (at 2.54 12.7) (size 1.7 1.7) (drill 1) (layers *.Cu *.Mask))
  (pad 10 thru_hole circle (at 2.54 10.16) (size 1.7 1.7) (drill 1) (layers *.Cu *.Mask))
  (pad 8 thru_hole circle (at 2.54 7.62) (size 1.7 1.7) (drill 1) (layers *.Cu *.Mask))
  (pad 6 thru_hole circle (at 2.54 5.08) (size 1.7 1.7) (drill 1) (layers *.Cu *.Mask))
  (pad 4 thru_hole circle (at 2.54 2.54) (size 1.7 1.7) (drill 1) (layers *.Cu *.Mask))
  (pad 2 thru_hole circle (at 2.54 0) (size 1.7 1.7) (drill 1) (layers *.Cu *.Mask))
  (pad 15 thru_hole circle (at 0 17.78) (size 1.7 1.7) (drill 1) (layers *.Cu *.Mask))
  (pad 13 thru_hole circle (at 0 15.24) (size 1.7 1.7) (drill 1) (layers *.Cu *.Mask))
  (pad 11 thru_hole circle (at 0 12.7) (size 1.7 1.7) (drill 1) (layers *.Cu *.Mask))
  (pad 9 thru_hole circle (at 0 10.16) (size 1.7 1.7) (drill 1) (layers *.Cu *.Mask))
  (pad 7 thru_hole circle (at 0 7.62) (size 1.7 1.7) (drill 1) (layers *.Cu *.Mask))
  (pad 5 thru_hole circle (at 0 5.08) (size 1.7 1.7) (drill 1) (layers *.Cu *.Mask))
  (pad 3 thru_hole circle (at 0 2.54) (size 1.7 1.7) (drill 1) (layers *.Cu *.Mask))
  (pad 1 thru_hole roundrect (at 0 0) (size 1.7 1.7) (drill 1) (layers *.Cu *.Mask) (roundrect_rratio 0.147059)))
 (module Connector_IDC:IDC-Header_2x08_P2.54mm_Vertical (layer F.Cu) (at 10.16 8.89)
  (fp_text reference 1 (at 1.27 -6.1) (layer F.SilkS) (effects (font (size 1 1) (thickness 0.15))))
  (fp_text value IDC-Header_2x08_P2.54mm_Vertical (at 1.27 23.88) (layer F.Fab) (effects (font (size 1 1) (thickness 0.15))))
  (pad 1 thru_hole roundrect (at 0 0) (size 1.7 1.7) (drill 1) (layers *.Cu *.Mask) (roundrect_rratio 0.147059))
  (pad 3 thru_hole circle (at 0 2.54) (size 1.7 1.7) (drill 1) (layers *.Cu *.Mask))
  (pad 5 thru_hole circle (at 0 5.08) (size 1.7 1.7) (drill 1) (layers *.Cu *.Mask))
  (pad 7 thru_hole circle (at 0 7.62) (size 1.7 1.7) (drill 1) (layers *.Cu *.Mask))
  (pad 9 thru_hole circle (at 0 10.16) (size 1.7 1.7) (drill 1) (layers *.Cu *.Mask))
  (pad 11 thru_hole circle (at 0 12.7) (size 1.7 1.7) (drill 1) (layers *.Cu *.Mask))
  (pad 13 thru_hole circle (at 0 15.24) (size 1.7 1.7) (drill 1) (layers *.Cu *.Mask))
  (pad 15 thru_hole circle (at 0 17.78) (size 1.7 1.7) (drill 1) (layers *.Cu *.Mask))
  (pad 2 thru_hole circle (at 2.54 0) (size 1.7 1.7) (drill 1) (layers *.Cu *.Mask))
  (pad 4 thru_hole circle (at 2.54 2.54) (size 1.7 1.7) (drill 1) (layers *.Cu *.Mask))
  (pad 6 thru_hole circle (at 2.54 5.08) (size 1.7 1.7) (drill 1) (layers *.Cu *.Mask))
  (pad 8 thru_hole circle (at 2.54 7.62) (size 1.7 1.7) (drill 1) (layers *.Cu *.Mask))
  (pad 10 thru_hole circle (at 2.54 10.16) (size 1.7 1.7) (drill 1) (layers *.Cu *.Mask))
  (pad 12 thru_hole circle (at 2.54 12.7) (size 1.7 1.7) (drill 1) (layers *.Cu *.Mask))
  (pad 14 thru_hole circle (at 2.54 15.24) (size 1.7 1.7) (drill 1) (layers *.Cu *.Mask))
  (pad 16 thru_hole circle (at 2.54 17.78) (size 1.7 1.7) (drill 1) (layers *.Cu *.Mask)))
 (gr_line (start 97.79 0) (end 97.79 69.85) (layer Edge.Cuts) (width 0.1))
 (gr_line (start 0 0) (end 97.79 0) (layer Edge.Cuts) (width 0.1))
 (gr_line (start 0 69.85) (end 0 0) (layer Edge.Cuts) (width 0.1))
 (gr_line (start 97.79 69.85) (end 0 69.85) (layer Edge.Cuts) (width 0.1))
 (segment (start 10.16 8.89) (end 12.7 8.89) (width 0.25) (layer F.Cu) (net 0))
 (segment (start 10.16 26.67) (end 12.7 26.67) (width 0.25) (layer F.Cu) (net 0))
 (segment (start 12.7 26.67) (end 22.86 26.67) (width 0.25) (layer F.Cu) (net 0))
 (segment (start 10.16 8.89) (end 88.9 8.89) (width 0.25) (layer F.Cu) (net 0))
 (segment (start 10.16 11.43) (end 88.9 11.43) (width 0.25) (layer F.Cu) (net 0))
 (segment (start 10.16 13.97) (end 17.78 13.97) (width 0.25) (layer F.Cu) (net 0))
 (segment (start 10.16 16.51) (end 30.48 16.51) (width 0.25) (layer F.Cu) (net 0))
 (segment (start 10.16 19.05) (end 43.18 19.05) (width 0.25) (layer F.Cu) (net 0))
 (segment (start 10.16 21.59) (end 55.88 21.59) (width 0.25) (layer F.Cu) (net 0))
 (segment (start 10.16 24.13) (end 68.58 24.13) (width 0.25) (layer F.Cu) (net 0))
 (segment (start 10.16 26.67) (end 81.28 26.67) (width 0.25) (layer F.Cu) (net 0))
 (segment (start 10.16 59.69) (end 81.28 59.69) (width 0.25) (layer F.Cu) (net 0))
 (segment (start 10.16 57.15) (end 68.58 57.15) (width 0.25) (layer F.Cu) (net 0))
 (segment (start 10.16 54.61) (end 55.88 54.61) (width 0.25) (layer F.Cu) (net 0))
 (segment (start 10.16 52.07) (end 43.18 52.07) (width 0.25) (layer F.Cu) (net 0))
 (segment (start 88.9 49.53) (end 30.48 49.53) (width 0.25) (layer F.Cu) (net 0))
 (segment (start 10.16 46.99) (end 17.78 46.99) (width 0.25) (layer F.Cu) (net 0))
 (segment (start 88.9 44.45) (end 10.16 44.45) (width 0.25) (layer F.Cu) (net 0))
 (segment (start 10.16 41.91) (end 88.9 41.91) (width 0.25) (layer F.Cu) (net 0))
 (segment (start 88.9 8.89) (end 95.25 8.89) (width 0.25) (layer F.Cu) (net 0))
 (segment (start 95.25 8.89) (end 95.25 41.91) (width 0.25) (layer F.Cu) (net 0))
 (segment (start 95.25 41.91) (end 88.9 41.91) (width 0.25) (layer F.Cu) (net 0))
 (segment (start 10.16 11.43) (end 2.54 11.43) (width 0.25) (layer F.Cu) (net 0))
 (segment (start 2.54 11.43) (end 2.54 44.45) (width 0.25) (layer F.Cu) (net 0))
 (segment (start 2.54 44.45) (end 10.16 44.45) (width 0.25) (layer F.Cu) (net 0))
 (segment (start 17.78 13.97) (end 88.9 13.97) (width 0.25) (layer F.Cu) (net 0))
 (via (at 17.78 13.97) (size 0.8) (drill 0.4) (layers F.Cu B.Cu) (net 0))
 (segment (start 17.78 46.99) (end 88.9 46.99) (width 0.25) (layer F.Cu) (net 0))
 (via (at 17.78 46.99) (size 0.8) (drill 0.4) (layers F.Cu B.Cu) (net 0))
 (segment (start 30.48 49.53) (end 10.16 49.53) (width 0.25) (layer F.Cu) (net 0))
 (via (at 30.48 49.53) (size 0.8) (drill 0.4) (layers F.Cu B.Cu) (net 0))
 (segment (start 30.48 16.51) (end 88.9 16.51) (width 0.25) (layer F.Cu) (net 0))
 (via (at 30.48 16.51) (size 0.8) (drill 0.4) (layers F.Cu B.Cu) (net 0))
 (segment (start 43.18 19.05) (end 88.9 19.05) (width 0.25) (layer F.Cu) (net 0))
 (via (at 43.18 19.05) (size 0.8) (drill 0.4) (layers F.Cu B.Cu) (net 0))
 (segment (start 43.18 52.07) (end 88.9 52.07) (width 0.25) (layer F.Cu) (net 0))
 (via (at 43.18 52.07) (size 0.8) (drill 0.4) (layers F.Cu B.Cu) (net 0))
 (segment (start 55.88 21.59) (end 88.9 21.59) (width 0.25) (layer F.Cu) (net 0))
 (via (at 55.88 21.59) (size 0.8) (drill 0.4) (layers F.Cu B.Cu) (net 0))
 (segment (start 55.88 54.61) (end 88.9 54.61) (width 0.25) (layer F.Cu) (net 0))
 (via (at 55.88 54.61) (size 0.8) (drill 0.4) (layers F.Cu B.Cu) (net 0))
 (segment (start 68.58 24.13) (end 88.9 24.13) (width 0.25) (layer F.Cu) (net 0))
 (via (at 68.58 24.13) (size 0.8) (drill 0.4) (layers F.Cu B.Cu) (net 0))
 (segment (start 68.58 57.15) (end 88.9 57.15) (width 0.25) (layer F.Cu) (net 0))
 (via (at 68.58 57.15) (size 0.8) (drill 0.4) (layers F.Cu B.Cu) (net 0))
 (segment (start 81.28 26.67) (end 88.9 26.67) (width 0.25) (layer F.Cu) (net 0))
 (via (at 81.28 26.67) (size 0.8) (drill 0.4) (layers F.Cu B.Cu) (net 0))
 (segment (start 81.28 59.69) (end 88.9 59.69) (width 0.25) (layer F.Cu) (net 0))
 (via (at 81.28 59.69) (size 0.8) (drill 0.4) (layers F.Cu B.Cu) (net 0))
 (segment (start 17.78 13.97) (end 17.78 46.99) (width 0.25) (layer B.Cu) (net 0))
 (segment (start 30.48 16.51) (end 30.48 49.53) (width 0.25) (layer B.Cu) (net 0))
 (segment (start 43.18 19.05) (end 43.18 52.07) (width 0.25) (layer B.Cu) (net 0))
 (segment (start 55.88 21.59) (end 55.88 54.61) (width 0.25) (layer B.Cu) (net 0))
 (segment (start 68.58 24.13) (end 68.58 57.15) (width 0.25) (layer B.Cu) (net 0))
 (segment (start 81.28 26.67) (end 81.28 59.69) (width 0.25) (layer B.Cu) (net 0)))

